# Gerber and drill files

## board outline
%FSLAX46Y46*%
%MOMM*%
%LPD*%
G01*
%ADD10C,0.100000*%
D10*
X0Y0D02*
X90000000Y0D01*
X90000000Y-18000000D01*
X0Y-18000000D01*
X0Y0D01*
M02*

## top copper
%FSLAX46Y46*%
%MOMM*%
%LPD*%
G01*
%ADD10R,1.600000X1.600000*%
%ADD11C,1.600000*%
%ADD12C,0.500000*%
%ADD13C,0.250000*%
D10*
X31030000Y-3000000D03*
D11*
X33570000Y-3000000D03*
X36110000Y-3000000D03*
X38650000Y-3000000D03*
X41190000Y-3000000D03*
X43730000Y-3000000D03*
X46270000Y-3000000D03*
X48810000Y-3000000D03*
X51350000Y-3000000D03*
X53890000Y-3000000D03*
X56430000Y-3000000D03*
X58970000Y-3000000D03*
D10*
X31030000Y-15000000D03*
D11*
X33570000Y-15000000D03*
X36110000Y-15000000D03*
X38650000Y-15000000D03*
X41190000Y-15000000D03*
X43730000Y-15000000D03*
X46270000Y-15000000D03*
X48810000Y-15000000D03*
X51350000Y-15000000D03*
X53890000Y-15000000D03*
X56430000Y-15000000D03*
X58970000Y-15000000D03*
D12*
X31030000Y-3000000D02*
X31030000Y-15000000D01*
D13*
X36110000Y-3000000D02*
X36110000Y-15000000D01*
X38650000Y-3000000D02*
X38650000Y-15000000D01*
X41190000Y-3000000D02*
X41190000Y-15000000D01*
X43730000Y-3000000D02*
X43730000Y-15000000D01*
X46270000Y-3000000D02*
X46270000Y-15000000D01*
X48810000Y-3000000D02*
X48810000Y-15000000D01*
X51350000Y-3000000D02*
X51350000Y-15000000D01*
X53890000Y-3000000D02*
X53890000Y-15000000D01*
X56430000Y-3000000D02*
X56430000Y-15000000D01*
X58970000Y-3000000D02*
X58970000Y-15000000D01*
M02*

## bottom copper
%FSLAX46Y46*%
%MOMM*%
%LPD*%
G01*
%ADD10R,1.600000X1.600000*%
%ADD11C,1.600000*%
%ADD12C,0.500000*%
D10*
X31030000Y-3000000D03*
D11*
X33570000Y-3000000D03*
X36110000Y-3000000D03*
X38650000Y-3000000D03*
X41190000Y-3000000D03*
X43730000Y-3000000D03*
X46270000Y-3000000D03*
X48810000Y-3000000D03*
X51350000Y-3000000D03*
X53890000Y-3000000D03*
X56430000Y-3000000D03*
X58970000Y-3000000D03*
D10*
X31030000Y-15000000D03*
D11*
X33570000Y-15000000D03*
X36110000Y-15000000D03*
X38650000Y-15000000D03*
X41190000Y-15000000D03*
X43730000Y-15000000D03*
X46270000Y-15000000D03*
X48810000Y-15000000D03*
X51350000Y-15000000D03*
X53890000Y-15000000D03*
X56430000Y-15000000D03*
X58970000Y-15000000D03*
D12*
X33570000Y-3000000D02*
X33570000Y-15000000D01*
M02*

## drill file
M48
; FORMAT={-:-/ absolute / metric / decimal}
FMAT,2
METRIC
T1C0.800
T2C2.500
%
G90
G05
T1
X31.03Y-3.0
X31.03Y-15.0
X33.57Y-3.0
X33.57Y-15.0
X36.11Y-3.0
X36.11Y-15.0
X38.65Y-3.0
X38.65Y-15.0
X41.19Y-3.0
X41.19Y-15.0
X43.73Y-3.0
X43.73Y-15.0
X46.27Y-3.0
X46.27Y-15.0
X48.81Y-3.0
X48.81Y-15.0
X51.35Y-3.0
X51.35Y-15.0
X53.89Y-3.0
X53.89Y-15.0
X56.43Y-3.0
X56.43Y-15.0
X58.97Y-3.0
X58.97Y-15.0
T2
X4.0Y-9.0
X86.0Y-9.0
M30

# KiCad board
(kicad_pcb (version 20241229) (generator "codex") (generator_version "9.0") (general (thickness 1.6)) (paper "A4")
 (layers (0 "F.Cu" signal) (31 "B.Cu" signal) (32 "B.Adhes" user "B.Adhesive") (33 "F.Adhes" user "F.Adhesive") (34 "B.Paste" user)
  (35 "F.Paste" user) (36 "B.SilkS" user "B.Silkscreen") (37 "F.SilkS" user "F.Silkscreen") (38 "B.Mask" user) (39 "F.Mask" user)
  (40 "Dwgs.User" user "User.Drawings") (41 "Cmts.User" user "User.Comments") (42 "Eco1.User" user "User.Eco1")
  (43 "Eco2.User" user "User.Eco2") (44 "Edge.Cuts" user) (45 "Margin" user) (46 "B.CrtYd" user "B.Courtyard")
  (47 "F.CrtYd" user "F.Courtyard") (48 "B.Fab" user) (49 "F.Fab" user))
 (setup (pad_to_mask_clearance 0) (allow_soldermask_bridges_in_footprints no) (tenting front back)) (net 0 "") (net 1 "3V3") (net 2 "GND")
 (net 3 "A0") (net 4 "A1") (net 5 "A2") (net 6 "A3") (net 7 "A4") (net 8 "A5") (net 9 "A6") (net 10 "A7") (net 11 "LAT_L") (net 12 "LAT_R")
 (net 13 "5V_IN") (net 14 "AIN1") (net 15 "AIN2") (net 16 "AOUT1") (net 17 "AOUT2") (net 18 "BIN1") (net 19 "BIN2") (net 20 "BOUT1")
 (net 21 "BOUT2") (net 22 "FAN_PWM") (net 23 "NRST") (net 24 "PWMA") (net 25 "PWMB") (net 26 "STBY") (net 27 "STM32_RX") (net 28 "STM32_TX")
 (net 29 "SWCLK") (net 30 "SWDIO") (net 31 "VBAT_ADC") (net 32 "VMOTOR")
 (gr_rect (start 0 0) (end 90 18) (stroke (width 0.1) (type solid)) (fill no) (layer "Edge.Cuts"))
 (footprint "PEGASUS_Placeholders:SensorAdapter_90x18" (layer "F.Cu") (at 45.000 9.000 0)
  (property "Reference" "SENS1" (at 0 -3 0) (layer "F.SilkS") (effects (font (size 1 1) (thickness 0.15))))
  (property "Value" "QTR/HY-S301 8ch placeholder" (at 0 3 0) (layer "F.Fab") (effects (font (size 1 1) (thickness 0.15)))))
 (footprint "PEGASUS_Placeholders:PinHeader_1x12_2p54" (layer "F.Cu") (at 45.000 3.000 0)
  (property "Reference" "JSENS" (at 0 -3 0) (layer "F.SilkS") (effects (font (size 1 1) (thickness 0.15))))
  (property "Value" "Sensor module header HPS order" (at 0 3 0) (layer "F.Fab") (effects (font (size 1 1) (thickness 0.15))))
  (pad "1" thru_hole rect (at -13.970 0.000) (size 1.6 1.6) (drill 0.8) (layers "*.Cu" "*.Mask") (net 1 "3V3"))
  (pad "2" thru_hole circle (at -11.430 0.000) (size 1.6 1.6) (drill 0.8) (layers "*.Cu" "*.Mask") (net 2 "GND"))
  (pad "3" thru_hole circle (at -8.890 0.000) (size 1.6 1.6) (drill 0.8) (layers "*.Cu" "*.Mask") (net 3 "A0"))
  (pad "4" thru_hole circle (at -6.350 0.000) (size 1.6 1.6) (drill 0.8) (layers "*.Cu" "*.Mask") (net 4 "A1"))
  (pad "5" thru_hole circle (at -3.810 0.000) (size 1.6 1.6) (drill 0.8) (layers "*.Cu" "*.Mask") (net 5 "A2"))
  (pad "6" thru_hole circle (at -1.270 0.000) (size 1.6 1.6) (drill 0.8) (layers "*.Cu" "*.Mask") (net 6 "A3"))
  (pad "7" thru_hole circle (at 1.270 0.000) (size 1.6 1.6) (drill 0.8) (layers "*.Cu" "*.Mask") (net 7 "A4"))
  (pad "8" thru_hole circle (at 3.810 0.000) (size 1.6 1.6) (drill 0.8) (layers "*.Cu" "*.Mask") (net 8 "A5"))
  (pad "9" thru_hole circle (at 6.350 0.000) (size 1.6 1.6) (drill 0.8) (layers "*.Cu" "*.Mask") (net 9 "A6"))
  (pad "10" thru_hole circle (at 8.890 0.000) (size 1.6 1.6) (drill 0.8) (layers "*.Cu" "*.Mask") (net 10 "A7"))
  (pad "11" thru_hole circle (at 11.430 0.000) (size 1.6 1.6) (drill 0.8) (layers "*.Cu" "*.Mask") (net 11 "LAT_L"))
  (pad "12" thru_hole circle (at 13.970 0.000) (size 1.6 1.6) (drill 0.8) (layers "*.Cu" "*.Mask") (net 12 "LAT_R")))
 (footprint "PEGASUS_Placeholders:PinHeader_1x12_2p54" (layer "F.Cu") (at 45.000 15.000 0)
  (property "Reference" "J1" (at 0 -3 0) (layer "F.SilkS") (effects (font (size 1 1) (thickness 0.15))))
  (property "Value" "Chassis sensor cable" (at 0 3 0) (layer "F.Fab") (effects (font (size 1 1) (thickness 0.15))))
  (pad "1" thru_hole rect (at -13.970 0.000) (size 1.6 1.6) (drill 0.8) (layers "*.Cu" "*.Mask") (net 1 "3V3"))
  (pad "2" thru_hole circle (at -11.430 0.000) (size 1.6 1.6) (drill 0.8) (layers "*.Cu" "*.Mask") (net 2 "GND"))
  (pad "3" thru_hole circle (at -8.890 0.000) (size 1.6 1.6) (drill 0.8) (layers "*.Cu" "*.Mask") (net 3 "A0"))
  (pad "4" thru_hole circle (at -6.350 0.000) (size 1.6 1.6) (drill 0.8) (layers "*.Cu" "*.Mask") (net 4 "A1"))
  (pad "5" thru_hole circle (at -3.810 0.000) (size 1.6 1.6) (drill 0.8) (layers "*.Cu" "*.Mask") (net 5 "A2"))
  (pad "6" thru_hole circle (at -1.270 0.000) (size 1.6 1.6) (drill 0.8) (layers "*.Cu" "*.Mask") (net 6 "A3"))
  (pad "7" thru_hole circle (at 1.270 0.000) (size 1.6 1.6) (drill 0.8) (layers "*.Cu" "*.Mask") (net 7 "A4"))
  (pad "8" thru_hole circle (at 3.810 0.000) (size 1.6 1.6) (drill 0.8) (layers "*.Cu" "*.Mask") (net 8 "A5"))
  (pad "9" thru_hole circle (at 6.350 0.000) (size 1.6 1.6) (drill 0.8) (layers "*.Cu" "*.Mask") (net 9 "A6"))
  (pad "10" thru_hole circle (at 8.890 0.000) (size 1.6 1.6) (drill 0.8) (layers "*.Cu" "*.Mask") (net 10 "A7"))
  (pad "11" thru_hole circle (at 11.430 0.000) (size 1.6 1.6) (drill 0.8) (layers "*.Cu" "*.Mask") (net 11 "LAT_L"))
  (pad "12" thru_hole circle (at 13.970 0.000) (size 1.6 1.6) (drill 0.8) (layers "*.Cu" "*.Mask") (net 12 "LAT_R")))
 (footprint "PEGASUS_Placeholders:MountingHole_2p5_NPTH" (layer "F.Cu") (at 4 9)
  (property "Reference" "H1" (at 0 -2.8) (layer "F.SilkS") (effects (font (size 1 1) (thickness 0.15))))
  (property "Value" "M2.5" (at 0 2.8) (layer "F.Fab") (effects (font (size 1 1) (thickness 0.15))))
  (pad "" np_thru_hole circle (at 0 0) (size 2.5 2.5) (drill 2.5) (layers "*.Cu" "*.Mask")))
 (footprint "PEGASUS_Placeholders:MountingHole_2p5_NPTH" (layer "F.Cu") (at 86 9)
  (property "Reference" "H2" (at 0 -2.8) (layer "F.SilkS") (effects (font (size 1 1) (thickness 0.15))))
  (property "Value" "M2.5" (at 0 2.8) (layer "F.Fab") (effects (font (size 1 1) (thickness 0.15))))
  (pad "" np_thru_hole circle (at 0 0) (size 2.5 2.5) (drill 2.5) (layers "*.Cu" "*.Mask")))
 (segment (start 31.030 3.000) (end 31.030 15.000) (width 0.50) (layer "F.Cu") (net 1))
 (segment (start 33.570 3.000) (end 33.570 15.000) (width 0.50) (layer "B.Cu") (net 2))
 (segment (start 36.110 3.000) (end 36.110 15.000) (width 0.25) (layer "F.Cu") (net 3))
 (segment (start 38.650 3.000) (end 38.650 15.000) (width 0.25) (layer "F.Cu") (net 4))
 (segment (start 41.190 3.000) (end 41.190 15.000) (width 0.25) (layer "F.Cu") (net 5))
 (segment (start 43.730 3.000) (end 43.730 15.000) (width 0.25) (layer "F.Cu") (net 6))
 (segment (start 46.270 3.000) (end 46.270 15.000) (width 0.25) (layer "F.Cu") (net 7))
 (segment (start 48.810 3.000) (end 48.810 15.000) (width 0.25) (layer "F.Cu") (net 8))
 (segment (start 51.350 3.000) (end 51.350 15.000) (width 0.25) (layer "F.Cu") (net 9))
 (segment (start 53.890 3.000) (end 53.890 15.000) (width 0.25) (layer "F.Cu") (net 10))
 (segment (start 56.430 3.000) (end 56.430 15.000) (width 0.25) (layer "F.Cu") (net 11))
 (segment (start 58.970 3.000) (end 58.970 15.000) (width 0.25) (layer "F.Cu") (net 12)))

